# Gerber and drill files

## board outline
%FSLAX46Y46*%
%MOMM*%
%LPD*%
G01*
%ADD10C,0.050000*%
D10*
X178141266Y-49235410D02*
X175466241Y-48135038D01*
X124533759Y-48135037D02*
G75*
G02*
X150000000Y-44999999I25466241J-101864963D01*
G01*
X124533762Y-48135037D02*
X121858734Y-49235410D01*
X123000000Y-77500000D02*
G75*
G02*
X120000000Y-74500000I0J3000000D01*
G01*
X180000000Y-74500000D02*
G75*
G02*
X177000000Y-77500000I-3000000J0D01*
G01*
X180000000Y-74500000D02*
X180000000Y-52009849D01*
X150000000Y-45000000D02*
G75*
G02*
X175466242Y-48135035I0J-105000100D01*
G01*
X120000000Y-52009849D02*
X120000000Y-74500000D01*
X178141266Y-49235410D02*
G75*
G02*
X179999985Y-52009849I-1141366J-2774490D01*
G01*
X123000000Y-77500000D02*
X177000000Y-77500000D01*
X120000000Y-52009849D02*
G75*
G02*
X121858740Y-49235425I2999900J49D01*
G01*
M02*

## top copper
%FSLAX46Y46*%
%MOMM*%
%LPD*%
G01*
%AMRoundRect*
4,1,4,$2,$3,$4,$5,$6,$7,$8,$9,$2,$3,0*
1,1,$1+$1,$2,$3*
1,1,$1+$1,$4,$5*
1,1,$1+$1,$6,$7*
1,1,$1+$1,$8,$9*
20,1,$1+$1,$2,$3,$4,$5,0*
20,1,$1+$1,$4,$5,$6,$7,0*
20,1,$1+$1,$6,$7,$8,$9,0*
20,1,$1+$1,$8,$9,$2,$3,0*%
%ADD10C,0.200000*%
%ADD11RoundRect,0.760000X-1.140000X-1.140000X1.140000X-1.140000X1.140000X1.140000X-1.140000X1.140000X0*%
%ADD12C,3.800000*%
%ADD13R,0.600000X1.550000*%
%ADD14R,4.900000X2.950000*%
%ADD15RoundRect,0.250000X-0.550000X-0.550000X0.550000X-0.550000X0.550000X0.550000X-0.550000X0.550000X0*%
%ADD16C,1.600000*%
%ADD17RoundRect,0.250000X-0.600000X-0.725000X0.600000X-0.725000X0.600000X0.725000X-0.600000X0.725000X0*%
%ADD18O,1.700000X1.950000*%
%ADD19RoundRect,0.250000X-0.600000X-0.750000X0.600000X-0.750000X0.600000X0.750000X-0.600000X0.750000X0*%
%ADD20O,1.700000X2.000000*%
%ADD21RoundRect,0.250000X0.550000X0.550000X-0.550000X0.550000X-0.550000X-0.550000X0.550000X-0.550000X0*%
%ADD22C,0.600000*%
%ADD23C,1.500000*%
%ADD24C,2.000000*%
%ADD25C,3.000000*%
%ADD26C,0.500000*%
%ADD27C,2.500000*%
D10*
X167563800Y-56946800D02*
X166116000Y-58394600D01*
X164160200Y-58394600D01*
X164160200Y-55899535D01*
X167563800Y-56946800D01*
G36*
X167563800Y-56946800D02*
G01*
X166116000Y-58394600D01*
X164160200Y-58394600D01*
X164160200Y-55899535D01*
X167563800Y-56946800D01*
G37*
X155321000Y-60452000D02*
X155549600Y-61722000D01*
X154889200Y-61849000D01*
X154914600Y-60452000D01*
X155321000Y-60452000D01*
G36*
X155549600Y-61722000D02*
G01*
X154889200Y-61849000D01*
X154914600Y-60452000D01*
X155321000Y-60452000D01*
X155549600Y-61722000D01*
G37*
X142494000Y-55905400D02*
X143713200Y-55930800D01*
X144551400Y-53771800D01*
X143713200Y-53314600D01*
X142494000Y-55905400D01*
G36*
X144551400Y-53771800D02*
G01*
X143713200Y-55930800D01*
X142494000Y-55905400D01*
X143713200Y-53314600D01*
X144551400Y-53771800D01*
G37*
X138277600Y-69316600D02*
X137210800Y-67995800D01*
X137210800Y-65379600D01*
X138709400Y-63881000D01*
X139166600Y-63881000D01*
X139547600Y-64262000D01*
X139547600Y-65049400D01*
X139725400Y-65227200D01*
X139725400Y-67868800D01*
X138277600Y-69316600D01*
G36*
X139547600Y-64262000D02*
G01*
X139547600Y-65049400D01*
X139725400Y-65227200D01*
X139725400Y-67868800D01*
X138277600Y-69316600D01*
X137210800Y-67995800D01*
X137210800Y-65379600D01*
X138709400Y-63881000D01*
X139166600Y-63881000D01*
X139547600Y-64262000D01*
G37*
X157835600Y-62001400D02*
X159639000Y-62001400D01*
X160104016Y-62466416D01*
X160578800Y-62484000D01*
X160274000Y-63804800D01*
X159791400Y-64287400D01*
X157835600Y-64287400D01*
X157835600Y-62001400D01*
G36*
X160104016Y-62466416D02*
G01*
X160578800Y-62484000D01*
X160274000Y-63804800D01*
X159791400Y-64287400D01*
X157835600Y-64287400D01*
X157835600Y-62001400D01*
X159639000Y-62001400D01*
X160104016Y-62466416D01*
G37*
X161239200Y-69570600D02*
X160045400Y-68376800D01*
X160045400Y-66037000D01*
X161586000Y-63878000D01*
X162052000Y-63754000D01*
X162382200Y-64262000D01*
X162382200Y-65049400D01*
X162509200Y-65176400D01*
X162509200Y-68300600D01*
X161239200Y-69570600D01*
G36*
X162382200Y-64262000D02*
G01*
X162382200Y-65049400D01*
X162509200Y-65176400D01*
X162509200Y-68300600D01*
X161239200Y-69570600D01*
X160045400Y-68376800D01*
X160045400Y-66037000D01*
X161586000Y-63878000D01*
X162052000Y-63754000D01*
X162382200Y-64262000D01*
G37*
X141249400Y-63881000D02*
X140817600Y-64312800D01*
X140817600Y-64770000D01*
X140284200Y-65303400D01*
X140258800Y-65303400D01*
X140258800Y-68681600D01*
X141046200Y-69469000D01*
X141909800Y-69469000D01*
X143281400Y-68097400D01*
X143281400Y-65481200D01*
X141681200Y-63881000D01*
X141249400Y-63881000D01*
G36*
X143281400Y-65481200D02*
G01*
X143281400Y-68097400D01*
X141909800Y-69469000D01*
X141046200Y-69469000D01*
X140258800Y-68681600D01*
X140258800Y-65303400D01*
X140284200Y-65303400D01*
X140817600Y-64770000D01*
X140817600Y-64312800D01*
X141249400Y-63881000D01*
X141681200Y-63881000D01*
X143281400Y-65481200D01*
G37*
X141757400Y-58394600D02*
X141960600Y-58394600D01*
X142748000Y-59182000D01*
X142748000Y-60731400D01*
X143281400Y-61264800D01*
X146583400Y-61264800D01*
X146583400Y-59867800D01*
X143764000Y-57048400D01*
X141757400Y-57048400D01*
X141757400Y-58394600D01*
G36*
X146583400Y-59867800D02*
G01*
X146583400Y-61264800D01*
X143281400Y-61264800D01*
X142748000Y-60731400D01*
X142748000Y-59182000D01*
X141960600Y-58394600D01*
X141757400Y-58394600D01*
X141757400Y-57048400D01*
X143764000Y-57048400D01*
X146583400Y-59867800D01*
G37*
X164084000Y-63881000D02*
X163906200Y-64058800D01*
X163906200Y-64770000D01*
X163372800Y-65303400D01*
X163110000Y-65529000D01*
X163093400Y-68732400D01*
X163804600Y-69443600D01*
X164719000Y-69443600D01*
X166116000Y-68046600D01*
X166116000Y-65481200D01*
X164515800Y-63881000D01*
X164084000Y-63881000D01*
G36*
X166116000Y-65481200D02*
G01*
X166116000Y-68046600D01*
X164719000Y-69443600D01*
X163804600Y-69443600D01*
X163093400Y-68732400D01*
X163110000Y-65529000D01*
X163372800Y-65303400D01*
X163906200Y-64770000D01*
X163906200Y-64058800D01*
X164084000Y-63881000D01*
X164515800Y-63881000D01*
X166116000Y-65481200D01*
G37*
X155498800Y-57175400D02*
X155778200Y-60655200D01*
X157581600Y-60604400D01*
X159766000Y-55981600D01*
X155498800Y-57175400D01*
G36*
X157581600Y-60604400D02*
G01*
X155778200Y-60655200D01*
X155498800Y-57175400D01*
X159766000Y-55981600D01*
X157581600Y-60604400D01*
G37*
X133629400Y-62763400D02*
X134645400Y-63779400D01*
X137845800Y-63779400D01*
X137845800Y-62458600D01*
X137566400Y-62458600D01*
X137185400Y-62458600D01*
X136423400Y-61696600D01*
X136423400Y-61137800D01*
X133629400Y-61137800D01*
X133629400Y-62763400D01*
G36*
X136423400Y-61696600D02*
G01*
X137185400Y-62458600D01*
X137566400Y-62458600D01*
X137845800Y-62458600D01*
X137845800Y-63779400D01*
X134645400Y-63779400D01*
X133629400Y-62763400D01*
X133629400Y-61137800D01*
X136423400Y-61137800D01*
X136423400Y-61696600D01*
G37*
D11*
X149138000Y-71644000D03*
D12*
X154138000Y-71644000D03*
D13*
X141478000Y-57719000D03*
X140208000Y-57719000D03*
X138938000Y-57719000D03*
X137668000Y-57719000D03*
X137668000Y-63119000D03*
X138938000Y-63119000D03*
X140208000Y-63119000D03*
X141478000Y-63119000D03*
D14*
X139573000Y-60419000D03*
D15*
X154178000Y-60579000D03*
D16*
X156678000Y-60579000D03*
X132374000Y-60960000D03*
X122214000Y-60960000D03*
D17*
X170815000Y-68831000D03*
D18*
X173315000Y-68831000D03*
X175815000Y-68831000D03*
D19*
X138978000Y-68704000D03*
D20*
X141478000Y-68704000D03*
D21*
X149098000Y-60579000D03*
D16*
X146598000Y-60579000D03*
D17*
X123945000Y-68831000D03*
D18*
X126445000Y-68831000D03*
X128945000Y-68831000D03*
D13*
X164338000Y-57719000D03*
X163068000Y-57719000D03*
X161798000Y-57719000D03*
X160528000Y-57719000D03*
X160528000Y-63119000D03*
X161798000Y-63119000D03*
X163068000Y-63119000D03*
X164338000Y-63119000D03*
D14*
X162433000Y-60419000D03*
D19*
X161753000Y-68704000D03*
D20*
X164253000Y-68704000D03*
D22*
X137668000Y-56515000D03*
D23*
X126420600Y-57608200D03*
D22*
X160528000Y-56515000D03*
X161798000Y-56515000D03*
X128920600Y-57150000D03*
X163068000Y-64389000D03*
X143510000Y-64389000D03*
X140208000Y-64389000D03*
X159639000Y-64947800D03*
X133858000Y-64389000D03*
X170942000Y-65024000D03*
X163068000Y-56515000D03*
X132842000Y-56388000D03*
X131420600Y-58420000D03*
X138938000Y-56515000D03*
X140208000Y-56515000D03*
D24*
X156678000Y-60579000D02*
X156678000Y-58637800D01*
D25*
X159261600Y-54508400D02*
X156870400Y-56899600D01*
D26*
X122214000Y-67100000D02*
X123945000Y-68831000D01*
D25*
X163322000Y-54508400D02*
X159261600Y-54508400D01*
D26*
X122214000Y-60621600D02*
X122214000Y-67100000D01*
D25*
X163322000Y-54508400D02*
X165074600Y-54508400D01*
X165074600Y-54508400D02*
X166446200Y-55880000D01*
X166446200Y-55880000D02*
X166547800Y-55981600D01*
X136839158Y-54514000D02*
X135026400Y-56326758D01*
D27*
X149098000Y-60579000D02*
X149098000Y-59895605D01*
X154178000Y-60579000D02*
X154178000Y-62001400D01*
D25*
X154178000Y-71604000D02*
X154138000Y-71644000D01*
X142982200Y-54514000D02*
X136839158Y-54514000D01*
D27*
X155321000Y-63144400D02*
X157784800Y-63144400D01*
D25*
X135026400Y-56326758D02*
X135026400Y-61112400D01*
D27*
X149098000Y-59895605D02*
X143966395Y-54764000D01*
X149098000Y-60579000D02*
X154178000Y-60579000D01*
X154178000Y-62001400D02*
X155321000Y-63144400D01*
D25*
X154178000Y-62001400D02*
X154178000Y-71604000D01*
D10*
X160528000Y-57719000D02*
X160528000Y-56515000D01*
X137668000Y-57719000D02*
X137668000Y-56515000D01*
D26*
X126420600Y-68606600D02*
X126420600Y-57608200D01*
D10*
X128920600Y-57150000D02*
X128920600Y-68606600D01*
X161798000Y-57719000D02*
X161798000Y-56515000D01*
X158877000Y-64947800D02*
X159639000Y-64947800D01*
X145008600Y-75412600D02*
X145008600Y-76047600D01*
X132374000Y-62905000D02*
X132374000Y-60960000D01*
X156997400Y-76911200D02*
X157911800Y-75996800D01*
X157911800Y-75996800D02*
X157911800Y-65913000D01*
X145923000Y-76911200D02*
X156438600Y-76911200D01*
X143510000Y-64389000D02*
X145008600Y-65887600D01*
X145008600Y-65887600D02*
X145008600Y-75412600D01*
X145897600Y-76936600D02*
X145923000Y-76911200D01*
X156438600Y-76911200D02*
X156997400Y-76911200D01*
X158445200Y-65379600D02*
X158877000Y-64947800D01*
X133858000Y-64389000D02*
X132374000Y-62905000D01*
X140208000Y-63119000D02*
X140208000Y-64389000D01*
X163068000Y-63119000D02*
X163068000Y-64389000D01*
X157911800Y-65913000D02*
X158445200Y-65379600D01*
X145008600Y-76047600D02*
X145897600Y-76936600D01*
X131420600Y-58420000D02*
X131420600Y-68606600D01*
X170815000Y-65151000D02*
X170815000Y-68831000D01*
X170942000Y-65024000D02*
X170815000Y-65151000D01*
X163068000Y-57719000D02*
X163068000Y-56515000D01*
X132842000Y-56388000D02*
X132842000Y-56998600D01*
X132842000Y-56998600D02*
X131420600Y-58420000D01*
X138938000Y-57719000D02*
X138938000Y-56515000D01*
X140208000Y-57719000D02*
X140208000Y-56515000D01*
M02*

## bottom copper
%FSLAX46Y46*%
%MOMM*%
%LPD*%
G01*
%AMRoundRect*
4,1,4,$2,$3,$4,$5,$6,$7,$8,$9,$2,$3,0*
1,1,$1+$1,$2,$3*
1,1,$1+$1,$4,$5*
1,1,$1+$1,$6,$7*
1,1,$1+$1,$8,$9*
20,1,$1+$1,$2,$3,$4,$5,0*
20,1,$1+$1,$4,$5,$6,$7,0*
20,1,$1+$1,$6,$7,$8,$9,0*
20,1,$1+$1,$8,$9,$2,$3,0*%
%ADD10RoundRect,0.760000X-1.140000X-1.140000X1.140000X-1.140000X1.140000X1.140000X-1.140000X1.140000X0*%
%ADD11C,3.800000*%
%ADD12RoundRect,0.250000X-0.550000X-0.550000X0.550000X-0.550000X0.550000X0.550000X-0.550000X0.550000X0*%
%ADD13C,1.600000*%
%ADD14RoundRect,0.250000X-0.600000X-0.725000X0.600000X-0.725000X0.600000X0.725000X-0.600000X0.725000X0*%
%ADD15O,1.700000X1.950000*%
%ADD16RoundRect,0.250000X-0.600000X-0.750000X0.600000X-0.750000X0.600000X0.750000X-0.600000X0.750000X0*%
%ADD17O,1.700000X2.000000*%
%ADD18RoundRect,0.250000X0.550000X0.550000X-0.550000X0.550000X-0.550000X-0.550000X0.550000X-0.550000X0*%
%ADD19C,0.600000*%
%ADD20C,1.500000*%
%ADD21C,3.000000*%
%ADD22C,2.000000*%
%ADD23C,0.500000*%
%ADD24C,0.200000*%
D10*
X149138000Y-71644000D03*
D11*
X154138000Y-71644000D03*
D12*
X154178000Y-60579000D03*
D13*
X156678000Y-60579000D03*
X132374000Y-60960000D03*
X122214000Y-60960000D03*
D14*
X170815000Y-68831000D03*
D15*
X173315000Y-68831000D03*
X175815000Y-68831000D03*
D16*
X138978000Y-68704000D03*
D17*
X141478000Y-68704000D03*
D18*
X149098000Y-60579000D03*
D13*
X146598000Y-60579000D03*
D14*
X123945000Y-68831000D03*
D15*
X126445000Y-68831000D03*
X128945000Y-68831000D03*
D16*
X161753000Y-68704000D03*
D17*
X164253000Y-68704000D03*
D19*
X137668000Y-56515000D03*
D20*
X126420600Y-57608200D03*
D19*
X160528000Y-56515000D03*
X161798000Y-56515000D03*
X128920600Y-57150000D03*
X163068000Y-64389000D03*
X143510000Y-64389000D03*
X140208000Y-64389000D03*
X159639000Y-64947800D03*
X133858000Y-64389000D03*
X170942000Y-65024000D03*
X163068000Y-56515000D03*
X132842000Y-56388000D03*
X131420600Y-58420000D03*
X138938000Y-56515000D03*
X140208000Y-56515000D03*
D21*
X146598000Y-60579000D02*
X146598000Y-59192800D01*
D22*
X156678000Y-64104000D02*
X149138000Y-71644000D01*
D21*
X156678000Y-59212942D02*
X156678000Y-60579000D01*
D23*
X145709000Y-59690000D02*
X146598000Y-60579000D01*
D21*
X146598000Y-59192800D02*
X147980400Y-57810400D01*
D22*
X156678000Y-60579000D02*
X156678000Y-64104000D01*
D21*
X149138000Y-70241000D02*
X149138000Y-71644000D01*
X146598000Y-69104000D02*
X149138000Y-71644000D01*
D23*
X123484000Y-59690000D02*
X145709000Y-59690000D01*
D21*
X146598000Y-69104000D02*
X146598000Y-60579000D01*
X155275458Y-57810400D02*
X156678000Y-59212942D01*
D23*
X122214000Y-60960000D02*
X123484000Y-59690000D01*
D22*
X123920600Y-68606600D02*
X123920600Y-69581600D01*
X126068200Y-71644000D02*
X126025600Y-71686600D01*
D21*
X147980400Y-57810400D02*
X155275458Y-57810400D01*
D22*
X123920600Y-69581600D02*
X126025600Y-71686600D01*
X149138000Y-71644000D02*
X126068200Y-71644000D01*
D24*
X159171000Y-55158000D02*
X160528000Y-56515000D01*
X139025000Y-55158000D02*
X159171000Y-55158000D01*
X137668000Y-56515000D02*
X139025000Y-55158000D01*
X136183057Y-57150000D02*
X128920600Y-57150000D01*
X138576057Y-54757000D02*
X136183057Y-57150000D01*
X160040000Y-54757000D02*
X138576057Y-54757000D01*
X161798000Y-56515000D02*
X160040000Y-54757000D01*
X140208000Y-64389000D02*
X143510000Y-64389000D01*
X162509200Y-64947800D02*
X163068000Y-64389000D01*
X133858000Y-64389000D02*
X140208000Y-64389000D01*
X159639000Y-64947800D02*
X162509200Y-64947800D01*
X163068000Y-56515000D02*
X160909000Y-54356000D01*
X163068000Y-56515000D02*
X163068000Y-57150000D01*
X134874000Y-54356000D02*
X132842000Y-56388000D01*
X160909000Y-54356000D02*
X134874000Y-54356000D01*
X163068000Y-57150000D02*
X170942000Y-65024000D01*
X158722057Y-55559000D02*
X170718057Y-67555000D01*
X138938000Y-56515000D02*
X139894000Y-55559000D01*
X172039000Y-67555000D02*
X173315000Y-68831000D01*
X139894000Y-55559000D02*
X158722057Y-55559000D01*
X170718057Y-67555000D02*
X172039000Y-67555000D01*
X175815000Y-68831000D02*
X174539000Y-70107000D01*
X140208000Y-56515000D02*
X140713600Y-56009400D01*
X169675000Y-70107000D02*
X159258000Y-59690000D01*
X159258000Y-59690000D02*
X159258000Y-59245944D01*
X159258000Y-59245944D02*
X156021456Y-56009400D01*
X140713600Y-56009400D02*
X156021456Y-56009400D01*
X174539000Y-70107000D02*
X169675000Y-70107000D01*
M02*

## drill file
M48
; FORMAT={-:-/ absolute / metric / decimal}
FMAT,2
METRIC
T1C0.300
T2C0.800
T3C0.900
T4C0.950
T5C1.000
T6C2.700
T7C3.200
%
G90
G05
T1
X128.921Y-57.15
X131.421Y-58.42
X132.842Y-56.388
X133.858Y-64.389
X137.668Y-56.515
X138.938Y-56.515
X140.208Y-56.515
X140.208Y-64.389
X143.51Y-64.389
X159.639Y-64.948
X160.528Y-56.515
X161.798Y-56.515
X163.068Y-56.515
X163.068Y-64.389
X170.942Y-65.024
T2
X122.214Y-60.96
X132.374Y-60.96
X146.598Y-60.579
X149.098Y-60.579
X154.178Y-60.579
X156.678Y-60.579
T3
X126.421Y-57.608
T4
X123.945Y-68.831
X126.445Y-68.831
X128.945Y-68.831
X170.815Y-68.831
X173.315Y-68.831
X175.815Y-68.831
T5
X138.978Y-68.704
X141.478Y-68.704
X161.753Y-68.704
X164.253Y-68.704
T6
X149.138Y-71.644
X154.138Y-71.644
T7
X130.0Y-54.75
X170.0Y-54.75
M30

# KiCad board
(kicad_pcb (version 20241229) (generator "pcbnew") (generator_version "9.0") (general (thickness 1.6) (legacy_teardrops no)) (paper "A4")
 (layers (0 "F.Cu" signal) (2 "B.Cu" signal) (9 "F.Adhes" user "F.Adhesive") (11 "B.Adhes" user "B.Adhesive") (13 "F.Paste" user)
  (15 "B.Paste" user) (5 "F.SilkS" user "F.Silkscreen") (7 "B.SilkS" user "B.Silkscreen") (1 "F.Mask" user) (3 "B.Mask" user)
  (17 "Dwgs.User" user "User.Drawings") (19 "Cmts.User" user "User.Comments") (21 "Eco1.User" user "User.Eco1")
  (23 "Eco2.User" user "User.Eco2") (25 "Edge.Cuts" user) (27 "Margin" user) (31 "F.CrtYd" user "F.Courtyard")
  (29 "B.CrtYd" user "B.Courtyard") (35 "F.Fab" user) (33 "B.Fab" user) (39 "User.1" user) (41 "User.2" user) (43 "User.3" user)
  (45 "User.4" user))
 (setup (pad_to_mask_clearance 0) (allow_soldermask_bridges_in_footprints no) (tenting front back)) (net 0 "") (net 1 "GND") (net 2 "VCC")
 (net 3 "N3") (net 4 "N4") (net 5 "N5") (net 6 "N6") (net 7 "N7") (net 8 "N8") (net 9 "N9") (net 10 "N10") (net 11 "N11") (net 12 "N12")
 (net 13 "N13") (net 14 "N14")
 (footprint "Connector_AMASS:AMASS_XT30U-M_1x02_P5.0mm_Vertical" (layer "F.Cu") (at 149.138 71.644)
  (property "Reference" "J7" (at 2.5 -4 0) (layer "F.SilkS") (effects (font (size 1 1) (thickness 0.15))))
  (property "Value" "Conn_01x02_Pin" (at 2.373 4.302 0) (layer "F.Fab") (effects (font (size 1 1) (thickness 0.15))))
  (pad "1" thru_hole roundrect (at 0 0) (size 3.8 3.8) (drill 2.7) (layers "*.Cu" "*.Mask") (remove_unused_layers no) (roundrect_rratio 0.2)
   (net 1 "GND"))
  (pad "2" thru_hole circle (at 5 0) (size 3.8 3.8) (drill 2.7) (layers "*.Cu" "*.Mask") (remove_unused_layers no) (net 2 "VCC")))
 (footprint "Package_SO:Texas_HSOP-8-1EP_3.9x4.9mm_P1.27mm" (layer "F.Cu") (at 139.573 60.419 -90)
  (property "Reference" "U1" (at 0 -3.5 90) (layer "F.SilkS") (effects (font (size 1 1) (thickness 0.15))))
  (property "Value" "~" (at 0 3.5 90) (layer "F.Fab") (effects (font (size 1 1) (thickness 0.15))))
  (pad "" smd rect (at 0 0 270) (size 2.6 3.1) (layers "F.Mask"))
  (pad "" smd rect (at 0 0 270) (size 2.6 3.1) (layers "F.Paste"))
  (pad "1" smd rect (at -2.7 -1.905 270) (size 1.55 0.6) (layers "F.Cu" "F.Mask" "F.Paste") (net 1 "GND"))
  (pad "2" smd rect (at -2.7 -0.635 270) (size 1.55 0.6) (layers "F.Cu" "F.Mask" "F.Paste") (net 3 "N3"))
  (pad "3" smd rect (at -2.7 0.635 270) (size 1.55 0.6) (layers "F.Cu" "F.Mask" "F.Paste") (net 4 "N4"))
  (pad "4" smd rect (at -2.7 1.905 270) (size 1.55 0.6) (layers "F.Cu" "F.Mask" "F.Paste") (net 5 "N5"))
  (pad "5" smd rect (at 2.7 1.905 270) (size 1.55 0.6) (layers "F.Cu" "F.Mask" "F.Paste") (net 2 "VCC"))
  (pad "6" smd rect (at 2.7 0.635 270) (size 1.55 0.6) (layers "F.Cu" "F.Mask" "F.Paste") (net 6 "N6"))
  (pad "7" smd rect (at 2.7 -0.635 270) (size 1.55 0.6) (layers "F.Cu" "F.Mask" "F.Paste") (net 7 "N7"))
  (pad "8" smd rect (at 2.7 -1.905 270) (size 1.55 0.6) (layers "F.Cu" "F.Mask" "F.Paste") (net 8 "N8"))
  (pad "9" smd rect (at 0 0 270) (size 2.95 4.9) (layers "F.Cu") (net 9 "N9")))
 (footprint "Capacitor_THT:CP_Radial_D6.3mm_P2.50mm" (layer "F.Cu") (at 154.178 60.579)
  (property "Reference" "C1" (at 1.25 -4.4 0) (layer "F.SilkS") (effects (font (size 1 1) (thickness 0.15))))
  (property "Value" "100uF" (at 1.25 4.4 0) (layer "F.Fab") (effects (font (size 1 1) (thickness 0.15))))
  (pad "1" thru_hole roundrect (at 0 0) (size 1.6 1.6) (drill 0.8) (layers "*.Cu" "*.Mask") (remove_unused_layers no)
   (roundrect_rratio 0.15625) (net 2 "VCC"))
  (pad "2" thru_hole circle (at 2.5 0) (size 1.6 1.6) (drill 0.8) (layers "*.Cu" "*.Mask") (remove_unused_layers no) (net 1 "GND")))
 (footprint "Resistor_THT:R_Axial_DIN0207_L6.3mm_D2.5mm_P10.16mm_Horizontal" (layer "F.Cu") (at 132.374 60.96 180)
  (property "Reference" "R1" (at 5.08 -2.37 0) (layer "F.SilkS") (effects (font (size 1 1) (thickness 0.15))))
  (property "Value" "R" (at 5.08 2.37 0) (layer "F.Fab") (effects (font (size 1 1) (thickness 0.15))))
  (pad "1" thru_hole circle (at 0 0 180) (size 1.6 1.6) (drill 0.8) (layers "*.Cu" "*.Mask") (remove_unused_layers no) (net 7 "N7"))
  (pad "2" thru_hole circle (at 10.16 0 180) (size 1.6 1.6) (drill 0.8) (layers "*.Cu" "*.Mask") (remove_unused_layers no) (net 1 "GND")))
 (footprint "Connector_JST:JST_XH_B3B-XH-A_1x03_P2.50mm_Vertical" (layer "F.Cu") (at 170.815 68.831)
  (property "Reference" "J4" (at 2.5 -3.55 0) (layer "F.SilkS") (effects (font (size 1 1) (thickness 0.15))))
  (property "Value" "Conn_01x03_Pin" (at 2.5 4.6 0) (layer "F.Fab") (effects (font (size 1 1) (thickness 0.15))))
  (pad "1" thru_hole roundrect (at 0 0) (size 1.7 1.95) (drill 0.95) (layers "*.Cu" "*.Mask") (remove_unused_layers no)
   (roundrect_rratio 0.147059) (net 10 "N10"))
  (pad "2" thru_hole oval (at 2.5 0) (size 1.7 1.95) (drill 0.95) (layers "*.Cu" "*.Mask") (remove_unused_layers no) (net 4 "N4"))
  (pad "3" thru_hole oval (at 5 0) (size 1.7 1.95) (drill 0.95) (layers "*.Cu" "*.Mask") (remove_unused_layers no) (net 3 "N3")))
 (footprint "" (layer "F.Cu") (at 130 54.75)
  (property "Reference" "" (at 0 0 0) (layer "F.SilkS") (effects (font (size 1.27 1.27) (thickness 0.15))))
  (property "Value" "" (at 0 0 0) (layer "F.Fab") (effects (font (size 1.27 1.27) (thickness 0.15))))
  (pad "" np_thru_hole circle (at 0 0) (size 3.2 3.2) (drill 3.2) (layers "*.Cu" "*.Mask")))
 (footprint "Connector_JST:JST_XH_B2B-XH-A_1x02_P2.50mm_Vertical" (layer "F.Cu") (at 138.978 68.704)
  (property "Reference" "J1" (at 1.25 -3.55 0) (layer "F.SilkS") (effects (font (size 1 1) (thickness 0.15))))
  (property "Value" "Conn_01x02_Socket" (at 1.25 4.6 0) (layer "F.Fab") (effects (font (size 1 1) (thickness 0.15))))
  (pad "1" thru_hole roundrect (at 0 0) (size 1.7 2) (drill 1) (layers "*.Cu" "*.Mask") (remove_unused_layers no)
   (roundrect_rratio 0.147059) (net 6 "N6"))
  (pad "2" thru_hole oval (at 2.5 0) (size 1.7 2) (drill 1) (layers "*.Cu" "*.Mask") (remove_unused_layers no) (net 8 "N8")))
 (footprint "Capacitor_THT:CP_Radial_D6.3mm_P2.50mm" (layer "F.Cu") (at 149.098 60.579 180)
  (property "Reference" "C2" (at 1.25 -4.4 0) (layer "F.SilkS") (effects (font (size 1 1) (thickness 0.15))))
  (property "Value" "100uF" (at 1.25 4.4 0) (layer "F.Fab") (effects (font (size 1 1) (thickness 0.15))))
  (pad "1" thru_hole roundrect (at 0 0 180) (size 1.6 1.6) (drill 0.8) (layers "*.Cu" "*.Mask") (remove_unused_layers no)
   (roundrect_rratio 0.15625) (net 2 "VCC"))
  (pad "2" thru_hole circle (at 2.5 0 180) (size 1.6 1.6) (drill 0.8) (layers "*.Cu" "*.Mask") (remove_unused_layers no) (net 1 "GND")))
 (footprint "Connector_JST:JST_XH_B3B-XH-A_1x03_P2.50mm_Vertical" (layer "F.Cu") (at 123.945 68.831)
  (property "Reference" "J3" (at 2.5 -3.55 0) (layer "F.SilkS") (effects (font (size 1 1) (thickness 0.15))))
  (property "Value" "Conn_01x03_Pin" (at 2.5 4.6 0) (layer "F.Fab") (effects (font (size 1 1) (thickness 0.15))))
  (pad "1" thru_hole roundrect (at 0 0) (size 1.7 1.95) (drill 0.95) (layers "*.Cu" "*.Mask") (remove_unused_layers no)
   (roundrect_rratio 0.147059) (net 1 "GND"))
  (pad "2" thru_hole oval (at 2.5 0) (size 1.7 1.95) (drill 0.95) (layers "*.Cu" "*.Mask") (remove_unused_layers no) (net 5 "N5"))
  (pad "3" thru_hole oval (at 5 0) (size 1.7 1.95) (drill 0.95) (layers "*.Cu" "*.Mask") (remove_unused_layers no) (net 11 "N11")))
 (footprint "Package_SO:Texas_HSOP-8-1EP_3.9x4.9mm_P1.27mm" (layer "F.Cu") (at 162.433 60.419 -90)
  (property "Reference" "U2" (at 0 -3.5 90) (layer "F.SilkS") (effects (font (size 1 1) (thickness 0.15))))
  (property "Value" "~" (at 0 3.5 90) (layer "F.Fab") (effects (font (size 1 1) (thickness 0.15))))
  (pad "" smd rect (at 0 0 270) (size 2.6 3.1) (layers "F.Mask"))
  (pad "" smd rect (at 0 0 270) (size 2.6 3.1) (layers "F.Paste"))
  (pad "1" smd rect (at -2.7 -1.905 270) (size 1.55 0.6) (layers "F.Cu" "F.Mask" "F.Paste") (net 1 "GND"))
  (pad "2" smd rect (at -2.7 -0.635 270) (size 1.55 0.6) (layers "F.Cu" "F.Mask" "F.Paste") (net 10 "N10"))
  (pad "3" smd rect (at -2.7 0.635 270) (size 1.55 0.6) (layers "F.Cu" "F.Mask" "F.Paste") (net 11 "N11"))
  (pad "4" smd rect (at -2.7 1.905 270) (size 1.55 0.6) (layers "F.Cu" "F.Mask" "F.Paste") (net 5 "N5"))
  (pad "5" smd rect (at 2.7 1.905 270) (size 1.55 0.6) (layers "F.Cu" "F.Mask" "F.Paste") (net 2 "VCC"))
  (pad "6" smd rect (at 2.7 0.635 270) (size 1.55 0.6) (layers "F.Cu" "F.Mask" "F.Paste") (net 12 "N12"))
  (pad "7" smd rect (at 2.7 -0.635 270) (size 1.55 0.6) (layers "F.Cu" "F.Mask" "F.Paste") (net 7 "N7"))
  (pad "8" smd rect (at 2.7 -1.905 270) (size 1.55 0.6) (layers "F.Cu" "F.Mask" "F.Paste") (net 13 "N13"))
  (pad "9" smd rect (at 0 0 270) (size 2.95 4.9) (layers "F.Cu") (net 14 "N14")))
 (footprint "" (layer "F.Cu") (at 170 54.75)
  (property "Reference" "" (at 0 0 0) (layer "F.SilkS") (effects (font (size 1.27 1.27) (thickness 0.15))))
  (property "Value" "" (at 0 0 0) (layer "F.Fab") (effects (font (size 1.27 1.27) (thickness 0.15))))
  (pad "" np_thru_hole circle (at 0 0) (size 3.2 3.2) (drill 3.2) (layers "*.Cu" "*.Mask")))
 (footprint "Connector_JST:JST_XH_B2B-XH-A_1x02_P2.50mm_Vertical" (layer "F.Cu") (at 161.753 68.704)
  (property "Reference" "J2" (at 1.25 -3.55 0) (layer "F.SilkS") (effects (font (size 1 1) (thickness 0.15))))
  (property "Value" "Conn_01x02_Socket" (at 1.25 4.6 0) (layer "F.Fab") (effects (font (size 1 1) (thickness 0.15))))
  (pad "1" thru_hole roundrect (at 0 0) (size 1.7 2) (drill 1) (layers "*.Cu" "*.Mask") (remove_unused_layers no)
   (roundrect_rratio 0.147059) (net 12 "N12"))
  (pad "2" thru_hole oval (at 2.5 0) (size 1.7 2) (drill 1) (layers "*.Cu" "*.Mask") (remove_unused_layers no) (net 13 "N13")))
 (gr_poly
  (pts (xy 167.5638 56.9468) (xy 166.116 58.3946) (xy 164.1602 58.3946) (xy 164.1602 55.899535)) (stroke (width 0.2) (type solid))
  (fill yes) (layer "F.Cu") (net 1))
 (gr_poly
  (pts (xy 155.321 60.452) (xy 155.5496 61.722) (xy 154.8892 61.849) (xy 154.9146 60.452)) (stroke (width 0.2) (type solid)) (fill yes)
  (layer "F.Cu") (net 2))
 (gr_poly
  (pts (xy 142.494 55.9054) (xy 143.7132 55.9308) (xy 144.5514 53.7718) (xy 143.7132 53.3146)) (stroke (width 0.2) (type solid)) (fill yes)
  (layer "F.Cu") (net 2))
 (gr_poly
  (pts (xy 138.2776 69.3166) (xy 137.2108 67.9958) (xy 137.2108 65.3796) (xy 138.7094 63.881) (xy 139.1666 63.881) (xy 139.5476 64.262)
   (xy 139.5476 65.0494) (xy 139.7254 65.2272) (xy 139.7254 67.8688))
  (stroke (width 0.2) (type solid)) (fill yes) (layer "F.Cu") (net 6))
 (gr_poly
  (pts (xy 157.8356 62.0014) (xy 159.639 62.0014) (xy 160.104016 62.466416) (xy 160.5788 62.484) (xy 160.274 63.8048) (xy 159.7914 64.2874)
   (xy 157.8356 64.2874))
  (stroke (width 0.2) (type solid)) (fill yes) (layer "F.Cu") (net 2))
 (gr_poly
  (pts (xy 161.2392 69.5706) (xy 160.0454 68.3768) (xy 160.0454 66.037) (xy 161.586 63.878) (xy 162.052 63.754) (xy 162.3822 64.262)
   (xy 162.3822 65.0494) (xy 162.5092 65.1764) (xy 162.5092 68.3006))
  (stroke (width 0.2) (type solid)) (fill yes) (layer "F.Cu") (net 12))
 (gr_poly
  (pts (xy 141.2494 63.881) (xy 140.8176 64.3128) (xy 140.8176 64.77) (xy 140.2842 65.3034) (xy 140.2588 65.3034) (xy 140.2588 68.6816)
   (xy 141.0462 69.469) (xy 141.9098 69.469) (xy 143.2814 68.0974) (xy 143.2814 65.4812) (xy 141.6812 63.881))
  (stroke (width 0.2) (type solid)) (fill yes) (layer "F.Cu") (net 8))
 (gr_poly
  (pts (xy 141.7574 58.3946) (xy 141.9606 58.3946) (xy 142.748 59.182) (xy 142.748 60.7314) (xy 143.2814 61.2648) (xy 146.5834 61.2648)
   (xy 146.5834 59.8678) (xy 143.764 57.0484) (xy 141.7574 57.0484))
  (stroke (width 0.2) (type solid)) (fill yes) (layer "F.Cu") (net 1))
 (gr_poly
  (pts (xy 164.084 63.881) (xy 163.9062 64.0588) (xy 163.9062 64.77) (xy 163.3728 65.3034) (xy 163.11 65.529) (xy 163.0934 68.7324)
   (xy 163.8046 69.4436) (xy 164.719 69.4436) (xy 166.116 68.0466) (xy 166.116 65.4812) (xy 164.5158 63.881))
  (stroke (width 0.2) (type solid)) (fill yes) (layer "F.Cu") (net 13))
 (gr_poly
  (pts (xy 155.4988 57.1754) (xy 155.7782 60.6552) (xy 157.5816 60.6044) (xy 159.766 55.9816)) (stroke (width 0.2) (type solid)) (fill yes)
  (layer "F.Cu") (net 1))
 (gr_poly
  (pts (xy 133.6294 62.7634) (xy 134.6454 63.7794) (xy 137.8458 63.7794) (xy 137.8458 62.4586) (xy 137.5664 62.4586) (xy 137.1854 62.4586)
   (xy 136.4234 61.6966) (xy 136.4234 61.1378) (xy 133.6294 61.1378))
  (stroke (width 0.2) (type solid)) (fill yes) (layer "F.Cu") (net 2))
 (gr_line (start 178.141266 49.23541) (end 175.466241 48.135038) (stroke (width 0.05) (type default)) (layer "Edge.Cuts"))
 (gr_arc (start 124.533759 48.135037) (mid 137.170757 45.786706) (end 150 45) (stroke (width 0.05) (type default)) (layer "Edge.Cuts"))
 (gr_line (start 124.533762 48.135037) (end 121.858734 49.23541) (stroke (width 0.05) (type default)) (layer "Edge.Cuts"))
 (gr_arc (start 123 77.5) (mid 120.87868 76.62132) (end 120 74.5) (stroke (width 0.05) (type default)) (layer "Edge.Cuts"))
 (gr_arc (start 180 74.5) (mid 179.12132 76.62132) (end 177 77.5) (stroke (width 0.05) (type default)) (layer "Edge.Cuts"))
 (gr_line (start 180 74.5) (end 180 52.009849) (stroke (width 0.05) (type default)) (layer "Edge.Cuts"))
 (gr_arc (start 150 45) (mid 162.829243 45.786707) (end 175.466241 48.135037) (stroke (width 0.05) (type default)) (layer "Edge.Cuts"))
 (gr_line (start 120 52.009849) (end 120 74.5) (stroke (width 0.05) (type default)) (layer "Edge.Cuts"))
 (gr_arc (start 178.141266 49.23541) (mid 179.492349 50.340093) (end 180 52.009849) (stroke (width 0.05) (type default)) (layer "Edge.Cuts"))
 (gr_line (start 123 77.5) (end 177 77.5) (stroke (width 0.05) (type default)) (layer "Edge.Cuts"))
 (gr_arc (start 120 52.009849) (mid 120.507613 50.340067) (end 121.858734 49.23541) (stroke (width 0.05) (type default)) (layer "Edge.Cuts"))
 (segment (start 156.678 60.579) (end 156.678 58.6378) (width 2) (layer "F.Cu") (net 1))
 (segment (start 159.2616 54.5084) (end 156.8704 56.8996) (width 3) (layer "F.Cu") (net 1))
 (segment (start 122.214 67.1) (end 123.945 68.831) (width 0.5) (layer "F.Cu") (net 1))
 (segment (start 163.322 54.5084) (end 159.2616 54.5084) (width 3) (layer "F.Cu") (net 1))
 (segment (start 122.214 60.6216) (end 122.214 67.1) (width 0.5) (layer "F.Cu") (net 1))
 (segment (start 163.322 54.5084) (end 165.0746 54.5084) (width 3) (layer "F.Cu") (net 1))
 (segment (start 165.0746 54.5084) (end 166.4462 55.88) (width 3) (layer "F.Cu") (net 1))
 (segment (start 166.4462 55.88) (end 166.5478 55.9816) (width 3) (layer "F.Cu") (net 1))
 (segment (start 146.598 60.579) (end 146.598 59.1928) (width 3) (layer "B.Cu") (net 1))
 (segment (start 156.678 64.104) (end 149.138 71.644) (width 2) (layer "B.Cu") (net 1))
 (segment (start 156.678 59.212942) (end 156.678 60.579) (width 3) (layer "B.Cu") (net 1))
 (segment (start 145.709 59.69) (end 146.598 60.579) (width 0.5) (layer "B.Cu") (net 1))
 (segment (start 146.598 59.1928) (end 147.9804 57.8104) (width 3) (layer "B.Cu") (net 1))
 (segment (start 156.678 60.579) (end 156.678 64.104) (width 2) (layer "B.Cu") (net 1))
 (segment (start 149.138 70.241) (end 149.138 71.644) (width 3) (layer "B.Cu") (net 1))
 (segment (start 146.598 69.104) (end 149.138 71.644) (width 3) (layer "B.Cu") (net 1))
 (segment (start 123.484 59.69) (end 145.709 59.69) (width 0.5) (layer "B.Cu") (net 1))
 (segment (start 146.598 69.104) (end 146.598 60.579) (width 3) (layer "B.Cu") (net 1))
 (segment (start 155.275458 57.8104) (end 156.678 59.212942) (width 3) (layer "B.Cu") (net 1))
 (segment (start 122.214 60.96) (end 123.484 59.69) (width 0.5) (layer "B.Cu") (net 1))
 (segment (start 123.9206 68.6066) (end 123.9206 69.5816) (width 2) (layer "B.Cu") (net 1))
 (segment (start 126.0682 71.644) (end 126.0256 71.6866) (width 2) (layer "B.Cu") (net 1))
 (segment (start 147.9804 57.8104) (end 155.275458 57.8104) (width 3) (layer "B.Cu") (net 1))
 (segment (start 123.9206 69.5816) (end 126.0256 71.6866) (width 2) (layer "B.Cu") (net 1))
 (segment (start 149.138 71.644) (end 126.0682 71.644) (width 2) (layer "B.Cu") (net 1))
 (segment (start 136.839158 54.514) (end 135.0264 56.326758) (width 3) (layer "F.Cu") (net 2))
 (segment (start 149.098 60.579) (end 149.098 59.895605) (width 2.5) (layer "F.Cu") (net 2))
 (segment (start 154.178 60.579) (end 154.178 62.0014) (width 2.5) (layer "F.Cu") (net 2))
 (segment (start 154.178 71.604) (end 154.138 71.644) (width 3) (layer "F.Cu") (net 2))
 (segment (start 142.9822 54.514) (end 136.839158 54.514) (width 3) (layer "F.Cu") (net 2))
 (segment (start 155.321 63.1444) (end 157.7848 63.1444) (width 2.5) (layer "F.Cu") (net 2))
 (segment (start 135.0264 56.326758) (end 135.0264 61.1124) (width 3) (layer "F.Cu") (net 2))
 (segment (start 149.098 59.895605) (end 143.966395 54.764) (width 2.5) (layer "F.Cu") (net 2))
 (segment (start 149.098 60.579) (end 154.178 60.579) (width 2.5) (layer "F.Cu") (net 2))
 (segment (start 154.178 62.0014) (end 155.321 63.1444) (width 2.5) (layer "F.Cu") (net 2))
 (segment (start 154.178 62.0014) (end 154.178 71.604) (width 3) (layer "F.Cu") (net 2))
 (segment (start 160.528 57.719) (end 160.528 56.515) (width 0.2) (layer "F.Cu") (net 5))
 (segment (start 137.668 57.719) (end 137.668 56.515) (width 0.2) (layer "F.Cu") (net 5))
 (segment (start 126.4206 68.6066) (end 126.4206 57.6082) (width 0.5) (layer "F.Cu") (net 5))
 (via (at 137.668 56.515) (size 0.6) (drill 0.3) (layers "F.Cu" "B.Cu") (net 5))
 (via (at 126.4206 57.6082) (size 1.5) (drill 0.9) (layers "F.Cu" "B.Cu") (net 5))
 (via (at 160.528 56.515) (size 0.6) (drill 0.3) (layers "F.Cu" "B.Cu") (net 5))
 (segment (start 159.171 55.158) (end 160.528 56.515) (width 0.2) (layer "B.Cu") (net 5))
 (segment (start 139.025 55.158) (end 159.171 55.158) (width 0.2) (layer "B.Cu") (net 5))
 (segment (start 137.668 56.515) (end 139.025 55.158) (width 0.2) (layer "B.Cu") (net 5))
 (segment (start 128.9206 57.15) (end 128.9206 68.6066) (width 0.2) (layer "F.Cu") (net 11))
 (segment (start 161.798 57.719) (end 161.798 56.515) (width 0.2) (layer "F.Cu") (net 11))
 (via (at 161.798 56.515) (size 0.6) (drill 0.3) (layers "F.Cu" "B.Cu") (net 11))
 (via (at 128.9206 57.15) (size 0.6) (drill 0.3) (layers "F.Cu" "B.Cu") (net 11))
 (segment (start 136.183057 57.15) (end 128.9206 57.15) (width 0.2) (layer "B.Cu") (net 11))
 (segment (start 138.576057 54.757) (end 136.183057 57.15) (width 0.2) (layer "B.Cu") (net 11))
 (segment (start 160.04 54.757) (end 138.576057 54.757) (width 0.2) (layer "B.Cu") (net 11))
 (segment (start 161.798 56.515) (end 160.04 54.757) (width 0.2) (layer "B.Cu") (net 11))
 (segment (start 158.877 64.9478) (end 159.639 64.9478) (width 0.2) (layer "F.Cu") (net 7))
 (segment (start 145.0086 75.4126) (end 145.0086 76.0476) (width 0.2) (layer "F.Cu") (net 7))
 (segment (start 132.374 62.905) (end 132.374 60.96) (width 0.2) (layer "F.Cu") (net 7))
 (segment (start 156.9974 76.9112) (end 157.9118 75.9968) (width 0.2) (layer "F.Cu") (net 7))
 (segment (start 157.9118 75.9968) (end 157.9118 65.913) (width 0.2) (layer "F.Cu") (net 7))
 (segment (start 145.923 76.9112) (end 156.4386 76.9112) (width 0.2) (layer "F.Cu") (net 7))
 (segment (start 143.51 64.389) (end 145.0086 65.8876) (width 0.2) (layer "F.Cu") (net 7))
 (segment (start 145.0086 65.8876) (end 145.0086 75.4126) (width 0.2) (layer "F.Cu") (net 7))
 (segment (start 145.8976 76.9366) (end 145.923 76.9112) (width 0.2) (layer "F.Cu") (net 7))
 (segment (start 156.4386 76.9112) (end 156.9974 76.9112) (width 0.2) (layer "F.Cu") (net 7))
 (segment (start 158.4452 65.3796) (end 158.877 64.9478) (width 0.2) (layer "F.Cu") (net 7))
 (segment (start 133.858 64.389) (end 132.374 62.905) (width 0.2) (layer "F.Cu") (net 7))
 (segment (start 140.208 63.119) (end 140.208 64.389) (width 0.2) (layer "F.Cu") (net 7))
 (segment (start 163.068 63.119) (end 163.068 64.389) (width 0.2) (layer "F.Cu") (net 7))
 (segment (start 157.9118 65.913) (end 158.4452 65.3796) (width 0.2) (layer "F.Cu") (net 7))
 (segment (start 145.0086 76.0476) (end 145.8976 76.9366) (width 0.2) (layer "F.Cu") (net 7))
 (via (at 163.068 64.389) (size 0.6) (drill 0.3) (layers "F.Cu" "B.Cu") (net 7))
 (via (at 143.51 64.389) (size 0.6) (drill 0.3) (layers "F.Cu" "B.Cu") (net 7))
 (via (at 140.208 64.389) (size 0.6) (drill 0.3) (layers "F.Cu" "B.Cu") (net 7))
 (via (at 159.639 64.9478) (size 0.6) (drill 0.3) (layers "F.Cu" "B.Cu") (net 7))
 (via (at 133.858 64.389) (size 0.6) (drill 0.3) (layers "F.Cu" "B.Cu") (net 7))
 (segment (start 140.208 64.389) (end 143.51 64.389) (width 0.2) (layer "B.Cu") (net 7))
 (segment (start 162.5092 64.9478) (end 163.068 64.389) (width 0.2) (layer "B.Cu") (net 7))
 (segment (start 133.858 64.389) (end 140.208 64.389) (width 0.2) (layer "B.Cu") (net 7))
 (segment (start 159.639 64.9478) (end 162.5092 64.9478) (width 0.2) (layer "B.Cu") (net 7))
 (segment (start 131.4206 58.42) (end 131.4206 68.6066) (width 0.2) (layer "F.Cu") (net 10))
 (segment (start 170.815 65.151) (end 170.815 68.831) (width 0.2) (layer "F.Cu") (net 10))
 (segment (start 170.942 65.024) (end 170.815 65.151) (width 0.2) (layer "F.Cu") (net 10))
 (segment (start 163.068 57.719) (end 163.068 56.515) (width 0.2) (layer "F.Cu") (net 10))
 (segment (start 132.842 56.388) (end 132.842 56.9986) (width 0.2) (layer "F.Cu") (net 10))
 (segment (start 132.842 56.9986) (end 131.4206 58.42) (width 0.2) (layer "F.Cu") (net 10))
 (via (at 170.942 65.024) (size 0.6) (drill 0.3) (layers "F.Cu" "B.Cu") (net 10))
 (via (at 163.068 56.515) (size 0.6) (drill 0.3) (layers "F.Cu" "B.Cu") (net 10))
 (via (at 132.842 56.388) (size 0.6) (drill 0.3) (layers "F.Cu" "B.Cu") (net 10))
 (via (at 131.4206 58.42) (size 0.6) (drill 0.3) (layers "F.Cu" "B.Cu") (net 10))
 (segment (start 163.068 56.515) (end 160.909 54.356) (width 0.2) (layer "B.Cu") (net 10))
 (segment (start 163.068 56.515) (end 163.068 57.15) (width 0.2) (layer "B.Cu") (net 10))
 (segment (start 134.874 54.356) (end 132.842 56.388) (width 0.2) (layer "B.Cu") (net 10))
 (segment (start 160.909 54.356) (end 134.874 54.356) (width 0.2) (layer "B.Cu") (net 10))
 (segment (start 163.068 57.15) (end 170.942 65.024) (width 0.2) (layer "B.Cu") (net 10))
 (segment (start 138.938 57.719) (end 138.938 56.515) (width 0.2) (layer "F.Cu") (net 4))
 (via (at 138.938 56.515) (size 0.6) (drill 0.3) (layers "F.Cu" "B.Cu") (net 4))
 (segment (start 158.722057 55.559) (end 170.718057 67.555) (width 0.2) (layer "B.Cu") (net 4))
 (segment (start 138.938 56.515) (end 139.894 55.559) (width 0.2) (layer "B.Cu") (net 4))
 (segment (start 172.039 67.555) (end 173.315 68.831) (width 0.2) (layer "B.Cu") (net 4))
 (segment (start 139.894 55.559) (end 158.722057 55.559) (width 0.2) (layer "B.Cu") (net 4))
 (segment (start 170.718057 67.555) (end 172.039 67.555) (width 0.2) (layer "B.Cu") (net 4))
 (segment (start 140.208 57.719) (end 140.208 56.515) (width 0.2) (layer "F.Cu") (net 3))
 (via (at 140.208 56.515) (size 0.6) (drill 0.3) (layers "F.Cu" "B.Cu") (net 3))
 (segment (start 175.815 68.831) (end 174.539 70.107) (width 0.2) (layer "B.Cu") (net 3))
 (segment (start 140.208 56.515) (end 140.7136 56.0094) (width 0.2) (layer "B.Cu") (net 3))
 (segment (start 169.675 70.107) (end 159.258 59.69) (width 0.2) (layer "B.Cu") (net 3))
 (segment (start 159.258 59.69) (end 159.258 59.245944) (width 0.2) (layer "B.Cu") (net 3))
 (segment (start 159.258 59.245944) (end 156.021456 56.0094) (width 0.2) (layer "B.Cu") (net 3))
 (segment (start 140.7136 56.0094) (end 156.021456 56.0094) (width 0.2) (layer "B.Cu") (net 3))
 (segment (start 174.539 70.107) (end 169.675 70.107) (width 0.2) (layer "B.Cu") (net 3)))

